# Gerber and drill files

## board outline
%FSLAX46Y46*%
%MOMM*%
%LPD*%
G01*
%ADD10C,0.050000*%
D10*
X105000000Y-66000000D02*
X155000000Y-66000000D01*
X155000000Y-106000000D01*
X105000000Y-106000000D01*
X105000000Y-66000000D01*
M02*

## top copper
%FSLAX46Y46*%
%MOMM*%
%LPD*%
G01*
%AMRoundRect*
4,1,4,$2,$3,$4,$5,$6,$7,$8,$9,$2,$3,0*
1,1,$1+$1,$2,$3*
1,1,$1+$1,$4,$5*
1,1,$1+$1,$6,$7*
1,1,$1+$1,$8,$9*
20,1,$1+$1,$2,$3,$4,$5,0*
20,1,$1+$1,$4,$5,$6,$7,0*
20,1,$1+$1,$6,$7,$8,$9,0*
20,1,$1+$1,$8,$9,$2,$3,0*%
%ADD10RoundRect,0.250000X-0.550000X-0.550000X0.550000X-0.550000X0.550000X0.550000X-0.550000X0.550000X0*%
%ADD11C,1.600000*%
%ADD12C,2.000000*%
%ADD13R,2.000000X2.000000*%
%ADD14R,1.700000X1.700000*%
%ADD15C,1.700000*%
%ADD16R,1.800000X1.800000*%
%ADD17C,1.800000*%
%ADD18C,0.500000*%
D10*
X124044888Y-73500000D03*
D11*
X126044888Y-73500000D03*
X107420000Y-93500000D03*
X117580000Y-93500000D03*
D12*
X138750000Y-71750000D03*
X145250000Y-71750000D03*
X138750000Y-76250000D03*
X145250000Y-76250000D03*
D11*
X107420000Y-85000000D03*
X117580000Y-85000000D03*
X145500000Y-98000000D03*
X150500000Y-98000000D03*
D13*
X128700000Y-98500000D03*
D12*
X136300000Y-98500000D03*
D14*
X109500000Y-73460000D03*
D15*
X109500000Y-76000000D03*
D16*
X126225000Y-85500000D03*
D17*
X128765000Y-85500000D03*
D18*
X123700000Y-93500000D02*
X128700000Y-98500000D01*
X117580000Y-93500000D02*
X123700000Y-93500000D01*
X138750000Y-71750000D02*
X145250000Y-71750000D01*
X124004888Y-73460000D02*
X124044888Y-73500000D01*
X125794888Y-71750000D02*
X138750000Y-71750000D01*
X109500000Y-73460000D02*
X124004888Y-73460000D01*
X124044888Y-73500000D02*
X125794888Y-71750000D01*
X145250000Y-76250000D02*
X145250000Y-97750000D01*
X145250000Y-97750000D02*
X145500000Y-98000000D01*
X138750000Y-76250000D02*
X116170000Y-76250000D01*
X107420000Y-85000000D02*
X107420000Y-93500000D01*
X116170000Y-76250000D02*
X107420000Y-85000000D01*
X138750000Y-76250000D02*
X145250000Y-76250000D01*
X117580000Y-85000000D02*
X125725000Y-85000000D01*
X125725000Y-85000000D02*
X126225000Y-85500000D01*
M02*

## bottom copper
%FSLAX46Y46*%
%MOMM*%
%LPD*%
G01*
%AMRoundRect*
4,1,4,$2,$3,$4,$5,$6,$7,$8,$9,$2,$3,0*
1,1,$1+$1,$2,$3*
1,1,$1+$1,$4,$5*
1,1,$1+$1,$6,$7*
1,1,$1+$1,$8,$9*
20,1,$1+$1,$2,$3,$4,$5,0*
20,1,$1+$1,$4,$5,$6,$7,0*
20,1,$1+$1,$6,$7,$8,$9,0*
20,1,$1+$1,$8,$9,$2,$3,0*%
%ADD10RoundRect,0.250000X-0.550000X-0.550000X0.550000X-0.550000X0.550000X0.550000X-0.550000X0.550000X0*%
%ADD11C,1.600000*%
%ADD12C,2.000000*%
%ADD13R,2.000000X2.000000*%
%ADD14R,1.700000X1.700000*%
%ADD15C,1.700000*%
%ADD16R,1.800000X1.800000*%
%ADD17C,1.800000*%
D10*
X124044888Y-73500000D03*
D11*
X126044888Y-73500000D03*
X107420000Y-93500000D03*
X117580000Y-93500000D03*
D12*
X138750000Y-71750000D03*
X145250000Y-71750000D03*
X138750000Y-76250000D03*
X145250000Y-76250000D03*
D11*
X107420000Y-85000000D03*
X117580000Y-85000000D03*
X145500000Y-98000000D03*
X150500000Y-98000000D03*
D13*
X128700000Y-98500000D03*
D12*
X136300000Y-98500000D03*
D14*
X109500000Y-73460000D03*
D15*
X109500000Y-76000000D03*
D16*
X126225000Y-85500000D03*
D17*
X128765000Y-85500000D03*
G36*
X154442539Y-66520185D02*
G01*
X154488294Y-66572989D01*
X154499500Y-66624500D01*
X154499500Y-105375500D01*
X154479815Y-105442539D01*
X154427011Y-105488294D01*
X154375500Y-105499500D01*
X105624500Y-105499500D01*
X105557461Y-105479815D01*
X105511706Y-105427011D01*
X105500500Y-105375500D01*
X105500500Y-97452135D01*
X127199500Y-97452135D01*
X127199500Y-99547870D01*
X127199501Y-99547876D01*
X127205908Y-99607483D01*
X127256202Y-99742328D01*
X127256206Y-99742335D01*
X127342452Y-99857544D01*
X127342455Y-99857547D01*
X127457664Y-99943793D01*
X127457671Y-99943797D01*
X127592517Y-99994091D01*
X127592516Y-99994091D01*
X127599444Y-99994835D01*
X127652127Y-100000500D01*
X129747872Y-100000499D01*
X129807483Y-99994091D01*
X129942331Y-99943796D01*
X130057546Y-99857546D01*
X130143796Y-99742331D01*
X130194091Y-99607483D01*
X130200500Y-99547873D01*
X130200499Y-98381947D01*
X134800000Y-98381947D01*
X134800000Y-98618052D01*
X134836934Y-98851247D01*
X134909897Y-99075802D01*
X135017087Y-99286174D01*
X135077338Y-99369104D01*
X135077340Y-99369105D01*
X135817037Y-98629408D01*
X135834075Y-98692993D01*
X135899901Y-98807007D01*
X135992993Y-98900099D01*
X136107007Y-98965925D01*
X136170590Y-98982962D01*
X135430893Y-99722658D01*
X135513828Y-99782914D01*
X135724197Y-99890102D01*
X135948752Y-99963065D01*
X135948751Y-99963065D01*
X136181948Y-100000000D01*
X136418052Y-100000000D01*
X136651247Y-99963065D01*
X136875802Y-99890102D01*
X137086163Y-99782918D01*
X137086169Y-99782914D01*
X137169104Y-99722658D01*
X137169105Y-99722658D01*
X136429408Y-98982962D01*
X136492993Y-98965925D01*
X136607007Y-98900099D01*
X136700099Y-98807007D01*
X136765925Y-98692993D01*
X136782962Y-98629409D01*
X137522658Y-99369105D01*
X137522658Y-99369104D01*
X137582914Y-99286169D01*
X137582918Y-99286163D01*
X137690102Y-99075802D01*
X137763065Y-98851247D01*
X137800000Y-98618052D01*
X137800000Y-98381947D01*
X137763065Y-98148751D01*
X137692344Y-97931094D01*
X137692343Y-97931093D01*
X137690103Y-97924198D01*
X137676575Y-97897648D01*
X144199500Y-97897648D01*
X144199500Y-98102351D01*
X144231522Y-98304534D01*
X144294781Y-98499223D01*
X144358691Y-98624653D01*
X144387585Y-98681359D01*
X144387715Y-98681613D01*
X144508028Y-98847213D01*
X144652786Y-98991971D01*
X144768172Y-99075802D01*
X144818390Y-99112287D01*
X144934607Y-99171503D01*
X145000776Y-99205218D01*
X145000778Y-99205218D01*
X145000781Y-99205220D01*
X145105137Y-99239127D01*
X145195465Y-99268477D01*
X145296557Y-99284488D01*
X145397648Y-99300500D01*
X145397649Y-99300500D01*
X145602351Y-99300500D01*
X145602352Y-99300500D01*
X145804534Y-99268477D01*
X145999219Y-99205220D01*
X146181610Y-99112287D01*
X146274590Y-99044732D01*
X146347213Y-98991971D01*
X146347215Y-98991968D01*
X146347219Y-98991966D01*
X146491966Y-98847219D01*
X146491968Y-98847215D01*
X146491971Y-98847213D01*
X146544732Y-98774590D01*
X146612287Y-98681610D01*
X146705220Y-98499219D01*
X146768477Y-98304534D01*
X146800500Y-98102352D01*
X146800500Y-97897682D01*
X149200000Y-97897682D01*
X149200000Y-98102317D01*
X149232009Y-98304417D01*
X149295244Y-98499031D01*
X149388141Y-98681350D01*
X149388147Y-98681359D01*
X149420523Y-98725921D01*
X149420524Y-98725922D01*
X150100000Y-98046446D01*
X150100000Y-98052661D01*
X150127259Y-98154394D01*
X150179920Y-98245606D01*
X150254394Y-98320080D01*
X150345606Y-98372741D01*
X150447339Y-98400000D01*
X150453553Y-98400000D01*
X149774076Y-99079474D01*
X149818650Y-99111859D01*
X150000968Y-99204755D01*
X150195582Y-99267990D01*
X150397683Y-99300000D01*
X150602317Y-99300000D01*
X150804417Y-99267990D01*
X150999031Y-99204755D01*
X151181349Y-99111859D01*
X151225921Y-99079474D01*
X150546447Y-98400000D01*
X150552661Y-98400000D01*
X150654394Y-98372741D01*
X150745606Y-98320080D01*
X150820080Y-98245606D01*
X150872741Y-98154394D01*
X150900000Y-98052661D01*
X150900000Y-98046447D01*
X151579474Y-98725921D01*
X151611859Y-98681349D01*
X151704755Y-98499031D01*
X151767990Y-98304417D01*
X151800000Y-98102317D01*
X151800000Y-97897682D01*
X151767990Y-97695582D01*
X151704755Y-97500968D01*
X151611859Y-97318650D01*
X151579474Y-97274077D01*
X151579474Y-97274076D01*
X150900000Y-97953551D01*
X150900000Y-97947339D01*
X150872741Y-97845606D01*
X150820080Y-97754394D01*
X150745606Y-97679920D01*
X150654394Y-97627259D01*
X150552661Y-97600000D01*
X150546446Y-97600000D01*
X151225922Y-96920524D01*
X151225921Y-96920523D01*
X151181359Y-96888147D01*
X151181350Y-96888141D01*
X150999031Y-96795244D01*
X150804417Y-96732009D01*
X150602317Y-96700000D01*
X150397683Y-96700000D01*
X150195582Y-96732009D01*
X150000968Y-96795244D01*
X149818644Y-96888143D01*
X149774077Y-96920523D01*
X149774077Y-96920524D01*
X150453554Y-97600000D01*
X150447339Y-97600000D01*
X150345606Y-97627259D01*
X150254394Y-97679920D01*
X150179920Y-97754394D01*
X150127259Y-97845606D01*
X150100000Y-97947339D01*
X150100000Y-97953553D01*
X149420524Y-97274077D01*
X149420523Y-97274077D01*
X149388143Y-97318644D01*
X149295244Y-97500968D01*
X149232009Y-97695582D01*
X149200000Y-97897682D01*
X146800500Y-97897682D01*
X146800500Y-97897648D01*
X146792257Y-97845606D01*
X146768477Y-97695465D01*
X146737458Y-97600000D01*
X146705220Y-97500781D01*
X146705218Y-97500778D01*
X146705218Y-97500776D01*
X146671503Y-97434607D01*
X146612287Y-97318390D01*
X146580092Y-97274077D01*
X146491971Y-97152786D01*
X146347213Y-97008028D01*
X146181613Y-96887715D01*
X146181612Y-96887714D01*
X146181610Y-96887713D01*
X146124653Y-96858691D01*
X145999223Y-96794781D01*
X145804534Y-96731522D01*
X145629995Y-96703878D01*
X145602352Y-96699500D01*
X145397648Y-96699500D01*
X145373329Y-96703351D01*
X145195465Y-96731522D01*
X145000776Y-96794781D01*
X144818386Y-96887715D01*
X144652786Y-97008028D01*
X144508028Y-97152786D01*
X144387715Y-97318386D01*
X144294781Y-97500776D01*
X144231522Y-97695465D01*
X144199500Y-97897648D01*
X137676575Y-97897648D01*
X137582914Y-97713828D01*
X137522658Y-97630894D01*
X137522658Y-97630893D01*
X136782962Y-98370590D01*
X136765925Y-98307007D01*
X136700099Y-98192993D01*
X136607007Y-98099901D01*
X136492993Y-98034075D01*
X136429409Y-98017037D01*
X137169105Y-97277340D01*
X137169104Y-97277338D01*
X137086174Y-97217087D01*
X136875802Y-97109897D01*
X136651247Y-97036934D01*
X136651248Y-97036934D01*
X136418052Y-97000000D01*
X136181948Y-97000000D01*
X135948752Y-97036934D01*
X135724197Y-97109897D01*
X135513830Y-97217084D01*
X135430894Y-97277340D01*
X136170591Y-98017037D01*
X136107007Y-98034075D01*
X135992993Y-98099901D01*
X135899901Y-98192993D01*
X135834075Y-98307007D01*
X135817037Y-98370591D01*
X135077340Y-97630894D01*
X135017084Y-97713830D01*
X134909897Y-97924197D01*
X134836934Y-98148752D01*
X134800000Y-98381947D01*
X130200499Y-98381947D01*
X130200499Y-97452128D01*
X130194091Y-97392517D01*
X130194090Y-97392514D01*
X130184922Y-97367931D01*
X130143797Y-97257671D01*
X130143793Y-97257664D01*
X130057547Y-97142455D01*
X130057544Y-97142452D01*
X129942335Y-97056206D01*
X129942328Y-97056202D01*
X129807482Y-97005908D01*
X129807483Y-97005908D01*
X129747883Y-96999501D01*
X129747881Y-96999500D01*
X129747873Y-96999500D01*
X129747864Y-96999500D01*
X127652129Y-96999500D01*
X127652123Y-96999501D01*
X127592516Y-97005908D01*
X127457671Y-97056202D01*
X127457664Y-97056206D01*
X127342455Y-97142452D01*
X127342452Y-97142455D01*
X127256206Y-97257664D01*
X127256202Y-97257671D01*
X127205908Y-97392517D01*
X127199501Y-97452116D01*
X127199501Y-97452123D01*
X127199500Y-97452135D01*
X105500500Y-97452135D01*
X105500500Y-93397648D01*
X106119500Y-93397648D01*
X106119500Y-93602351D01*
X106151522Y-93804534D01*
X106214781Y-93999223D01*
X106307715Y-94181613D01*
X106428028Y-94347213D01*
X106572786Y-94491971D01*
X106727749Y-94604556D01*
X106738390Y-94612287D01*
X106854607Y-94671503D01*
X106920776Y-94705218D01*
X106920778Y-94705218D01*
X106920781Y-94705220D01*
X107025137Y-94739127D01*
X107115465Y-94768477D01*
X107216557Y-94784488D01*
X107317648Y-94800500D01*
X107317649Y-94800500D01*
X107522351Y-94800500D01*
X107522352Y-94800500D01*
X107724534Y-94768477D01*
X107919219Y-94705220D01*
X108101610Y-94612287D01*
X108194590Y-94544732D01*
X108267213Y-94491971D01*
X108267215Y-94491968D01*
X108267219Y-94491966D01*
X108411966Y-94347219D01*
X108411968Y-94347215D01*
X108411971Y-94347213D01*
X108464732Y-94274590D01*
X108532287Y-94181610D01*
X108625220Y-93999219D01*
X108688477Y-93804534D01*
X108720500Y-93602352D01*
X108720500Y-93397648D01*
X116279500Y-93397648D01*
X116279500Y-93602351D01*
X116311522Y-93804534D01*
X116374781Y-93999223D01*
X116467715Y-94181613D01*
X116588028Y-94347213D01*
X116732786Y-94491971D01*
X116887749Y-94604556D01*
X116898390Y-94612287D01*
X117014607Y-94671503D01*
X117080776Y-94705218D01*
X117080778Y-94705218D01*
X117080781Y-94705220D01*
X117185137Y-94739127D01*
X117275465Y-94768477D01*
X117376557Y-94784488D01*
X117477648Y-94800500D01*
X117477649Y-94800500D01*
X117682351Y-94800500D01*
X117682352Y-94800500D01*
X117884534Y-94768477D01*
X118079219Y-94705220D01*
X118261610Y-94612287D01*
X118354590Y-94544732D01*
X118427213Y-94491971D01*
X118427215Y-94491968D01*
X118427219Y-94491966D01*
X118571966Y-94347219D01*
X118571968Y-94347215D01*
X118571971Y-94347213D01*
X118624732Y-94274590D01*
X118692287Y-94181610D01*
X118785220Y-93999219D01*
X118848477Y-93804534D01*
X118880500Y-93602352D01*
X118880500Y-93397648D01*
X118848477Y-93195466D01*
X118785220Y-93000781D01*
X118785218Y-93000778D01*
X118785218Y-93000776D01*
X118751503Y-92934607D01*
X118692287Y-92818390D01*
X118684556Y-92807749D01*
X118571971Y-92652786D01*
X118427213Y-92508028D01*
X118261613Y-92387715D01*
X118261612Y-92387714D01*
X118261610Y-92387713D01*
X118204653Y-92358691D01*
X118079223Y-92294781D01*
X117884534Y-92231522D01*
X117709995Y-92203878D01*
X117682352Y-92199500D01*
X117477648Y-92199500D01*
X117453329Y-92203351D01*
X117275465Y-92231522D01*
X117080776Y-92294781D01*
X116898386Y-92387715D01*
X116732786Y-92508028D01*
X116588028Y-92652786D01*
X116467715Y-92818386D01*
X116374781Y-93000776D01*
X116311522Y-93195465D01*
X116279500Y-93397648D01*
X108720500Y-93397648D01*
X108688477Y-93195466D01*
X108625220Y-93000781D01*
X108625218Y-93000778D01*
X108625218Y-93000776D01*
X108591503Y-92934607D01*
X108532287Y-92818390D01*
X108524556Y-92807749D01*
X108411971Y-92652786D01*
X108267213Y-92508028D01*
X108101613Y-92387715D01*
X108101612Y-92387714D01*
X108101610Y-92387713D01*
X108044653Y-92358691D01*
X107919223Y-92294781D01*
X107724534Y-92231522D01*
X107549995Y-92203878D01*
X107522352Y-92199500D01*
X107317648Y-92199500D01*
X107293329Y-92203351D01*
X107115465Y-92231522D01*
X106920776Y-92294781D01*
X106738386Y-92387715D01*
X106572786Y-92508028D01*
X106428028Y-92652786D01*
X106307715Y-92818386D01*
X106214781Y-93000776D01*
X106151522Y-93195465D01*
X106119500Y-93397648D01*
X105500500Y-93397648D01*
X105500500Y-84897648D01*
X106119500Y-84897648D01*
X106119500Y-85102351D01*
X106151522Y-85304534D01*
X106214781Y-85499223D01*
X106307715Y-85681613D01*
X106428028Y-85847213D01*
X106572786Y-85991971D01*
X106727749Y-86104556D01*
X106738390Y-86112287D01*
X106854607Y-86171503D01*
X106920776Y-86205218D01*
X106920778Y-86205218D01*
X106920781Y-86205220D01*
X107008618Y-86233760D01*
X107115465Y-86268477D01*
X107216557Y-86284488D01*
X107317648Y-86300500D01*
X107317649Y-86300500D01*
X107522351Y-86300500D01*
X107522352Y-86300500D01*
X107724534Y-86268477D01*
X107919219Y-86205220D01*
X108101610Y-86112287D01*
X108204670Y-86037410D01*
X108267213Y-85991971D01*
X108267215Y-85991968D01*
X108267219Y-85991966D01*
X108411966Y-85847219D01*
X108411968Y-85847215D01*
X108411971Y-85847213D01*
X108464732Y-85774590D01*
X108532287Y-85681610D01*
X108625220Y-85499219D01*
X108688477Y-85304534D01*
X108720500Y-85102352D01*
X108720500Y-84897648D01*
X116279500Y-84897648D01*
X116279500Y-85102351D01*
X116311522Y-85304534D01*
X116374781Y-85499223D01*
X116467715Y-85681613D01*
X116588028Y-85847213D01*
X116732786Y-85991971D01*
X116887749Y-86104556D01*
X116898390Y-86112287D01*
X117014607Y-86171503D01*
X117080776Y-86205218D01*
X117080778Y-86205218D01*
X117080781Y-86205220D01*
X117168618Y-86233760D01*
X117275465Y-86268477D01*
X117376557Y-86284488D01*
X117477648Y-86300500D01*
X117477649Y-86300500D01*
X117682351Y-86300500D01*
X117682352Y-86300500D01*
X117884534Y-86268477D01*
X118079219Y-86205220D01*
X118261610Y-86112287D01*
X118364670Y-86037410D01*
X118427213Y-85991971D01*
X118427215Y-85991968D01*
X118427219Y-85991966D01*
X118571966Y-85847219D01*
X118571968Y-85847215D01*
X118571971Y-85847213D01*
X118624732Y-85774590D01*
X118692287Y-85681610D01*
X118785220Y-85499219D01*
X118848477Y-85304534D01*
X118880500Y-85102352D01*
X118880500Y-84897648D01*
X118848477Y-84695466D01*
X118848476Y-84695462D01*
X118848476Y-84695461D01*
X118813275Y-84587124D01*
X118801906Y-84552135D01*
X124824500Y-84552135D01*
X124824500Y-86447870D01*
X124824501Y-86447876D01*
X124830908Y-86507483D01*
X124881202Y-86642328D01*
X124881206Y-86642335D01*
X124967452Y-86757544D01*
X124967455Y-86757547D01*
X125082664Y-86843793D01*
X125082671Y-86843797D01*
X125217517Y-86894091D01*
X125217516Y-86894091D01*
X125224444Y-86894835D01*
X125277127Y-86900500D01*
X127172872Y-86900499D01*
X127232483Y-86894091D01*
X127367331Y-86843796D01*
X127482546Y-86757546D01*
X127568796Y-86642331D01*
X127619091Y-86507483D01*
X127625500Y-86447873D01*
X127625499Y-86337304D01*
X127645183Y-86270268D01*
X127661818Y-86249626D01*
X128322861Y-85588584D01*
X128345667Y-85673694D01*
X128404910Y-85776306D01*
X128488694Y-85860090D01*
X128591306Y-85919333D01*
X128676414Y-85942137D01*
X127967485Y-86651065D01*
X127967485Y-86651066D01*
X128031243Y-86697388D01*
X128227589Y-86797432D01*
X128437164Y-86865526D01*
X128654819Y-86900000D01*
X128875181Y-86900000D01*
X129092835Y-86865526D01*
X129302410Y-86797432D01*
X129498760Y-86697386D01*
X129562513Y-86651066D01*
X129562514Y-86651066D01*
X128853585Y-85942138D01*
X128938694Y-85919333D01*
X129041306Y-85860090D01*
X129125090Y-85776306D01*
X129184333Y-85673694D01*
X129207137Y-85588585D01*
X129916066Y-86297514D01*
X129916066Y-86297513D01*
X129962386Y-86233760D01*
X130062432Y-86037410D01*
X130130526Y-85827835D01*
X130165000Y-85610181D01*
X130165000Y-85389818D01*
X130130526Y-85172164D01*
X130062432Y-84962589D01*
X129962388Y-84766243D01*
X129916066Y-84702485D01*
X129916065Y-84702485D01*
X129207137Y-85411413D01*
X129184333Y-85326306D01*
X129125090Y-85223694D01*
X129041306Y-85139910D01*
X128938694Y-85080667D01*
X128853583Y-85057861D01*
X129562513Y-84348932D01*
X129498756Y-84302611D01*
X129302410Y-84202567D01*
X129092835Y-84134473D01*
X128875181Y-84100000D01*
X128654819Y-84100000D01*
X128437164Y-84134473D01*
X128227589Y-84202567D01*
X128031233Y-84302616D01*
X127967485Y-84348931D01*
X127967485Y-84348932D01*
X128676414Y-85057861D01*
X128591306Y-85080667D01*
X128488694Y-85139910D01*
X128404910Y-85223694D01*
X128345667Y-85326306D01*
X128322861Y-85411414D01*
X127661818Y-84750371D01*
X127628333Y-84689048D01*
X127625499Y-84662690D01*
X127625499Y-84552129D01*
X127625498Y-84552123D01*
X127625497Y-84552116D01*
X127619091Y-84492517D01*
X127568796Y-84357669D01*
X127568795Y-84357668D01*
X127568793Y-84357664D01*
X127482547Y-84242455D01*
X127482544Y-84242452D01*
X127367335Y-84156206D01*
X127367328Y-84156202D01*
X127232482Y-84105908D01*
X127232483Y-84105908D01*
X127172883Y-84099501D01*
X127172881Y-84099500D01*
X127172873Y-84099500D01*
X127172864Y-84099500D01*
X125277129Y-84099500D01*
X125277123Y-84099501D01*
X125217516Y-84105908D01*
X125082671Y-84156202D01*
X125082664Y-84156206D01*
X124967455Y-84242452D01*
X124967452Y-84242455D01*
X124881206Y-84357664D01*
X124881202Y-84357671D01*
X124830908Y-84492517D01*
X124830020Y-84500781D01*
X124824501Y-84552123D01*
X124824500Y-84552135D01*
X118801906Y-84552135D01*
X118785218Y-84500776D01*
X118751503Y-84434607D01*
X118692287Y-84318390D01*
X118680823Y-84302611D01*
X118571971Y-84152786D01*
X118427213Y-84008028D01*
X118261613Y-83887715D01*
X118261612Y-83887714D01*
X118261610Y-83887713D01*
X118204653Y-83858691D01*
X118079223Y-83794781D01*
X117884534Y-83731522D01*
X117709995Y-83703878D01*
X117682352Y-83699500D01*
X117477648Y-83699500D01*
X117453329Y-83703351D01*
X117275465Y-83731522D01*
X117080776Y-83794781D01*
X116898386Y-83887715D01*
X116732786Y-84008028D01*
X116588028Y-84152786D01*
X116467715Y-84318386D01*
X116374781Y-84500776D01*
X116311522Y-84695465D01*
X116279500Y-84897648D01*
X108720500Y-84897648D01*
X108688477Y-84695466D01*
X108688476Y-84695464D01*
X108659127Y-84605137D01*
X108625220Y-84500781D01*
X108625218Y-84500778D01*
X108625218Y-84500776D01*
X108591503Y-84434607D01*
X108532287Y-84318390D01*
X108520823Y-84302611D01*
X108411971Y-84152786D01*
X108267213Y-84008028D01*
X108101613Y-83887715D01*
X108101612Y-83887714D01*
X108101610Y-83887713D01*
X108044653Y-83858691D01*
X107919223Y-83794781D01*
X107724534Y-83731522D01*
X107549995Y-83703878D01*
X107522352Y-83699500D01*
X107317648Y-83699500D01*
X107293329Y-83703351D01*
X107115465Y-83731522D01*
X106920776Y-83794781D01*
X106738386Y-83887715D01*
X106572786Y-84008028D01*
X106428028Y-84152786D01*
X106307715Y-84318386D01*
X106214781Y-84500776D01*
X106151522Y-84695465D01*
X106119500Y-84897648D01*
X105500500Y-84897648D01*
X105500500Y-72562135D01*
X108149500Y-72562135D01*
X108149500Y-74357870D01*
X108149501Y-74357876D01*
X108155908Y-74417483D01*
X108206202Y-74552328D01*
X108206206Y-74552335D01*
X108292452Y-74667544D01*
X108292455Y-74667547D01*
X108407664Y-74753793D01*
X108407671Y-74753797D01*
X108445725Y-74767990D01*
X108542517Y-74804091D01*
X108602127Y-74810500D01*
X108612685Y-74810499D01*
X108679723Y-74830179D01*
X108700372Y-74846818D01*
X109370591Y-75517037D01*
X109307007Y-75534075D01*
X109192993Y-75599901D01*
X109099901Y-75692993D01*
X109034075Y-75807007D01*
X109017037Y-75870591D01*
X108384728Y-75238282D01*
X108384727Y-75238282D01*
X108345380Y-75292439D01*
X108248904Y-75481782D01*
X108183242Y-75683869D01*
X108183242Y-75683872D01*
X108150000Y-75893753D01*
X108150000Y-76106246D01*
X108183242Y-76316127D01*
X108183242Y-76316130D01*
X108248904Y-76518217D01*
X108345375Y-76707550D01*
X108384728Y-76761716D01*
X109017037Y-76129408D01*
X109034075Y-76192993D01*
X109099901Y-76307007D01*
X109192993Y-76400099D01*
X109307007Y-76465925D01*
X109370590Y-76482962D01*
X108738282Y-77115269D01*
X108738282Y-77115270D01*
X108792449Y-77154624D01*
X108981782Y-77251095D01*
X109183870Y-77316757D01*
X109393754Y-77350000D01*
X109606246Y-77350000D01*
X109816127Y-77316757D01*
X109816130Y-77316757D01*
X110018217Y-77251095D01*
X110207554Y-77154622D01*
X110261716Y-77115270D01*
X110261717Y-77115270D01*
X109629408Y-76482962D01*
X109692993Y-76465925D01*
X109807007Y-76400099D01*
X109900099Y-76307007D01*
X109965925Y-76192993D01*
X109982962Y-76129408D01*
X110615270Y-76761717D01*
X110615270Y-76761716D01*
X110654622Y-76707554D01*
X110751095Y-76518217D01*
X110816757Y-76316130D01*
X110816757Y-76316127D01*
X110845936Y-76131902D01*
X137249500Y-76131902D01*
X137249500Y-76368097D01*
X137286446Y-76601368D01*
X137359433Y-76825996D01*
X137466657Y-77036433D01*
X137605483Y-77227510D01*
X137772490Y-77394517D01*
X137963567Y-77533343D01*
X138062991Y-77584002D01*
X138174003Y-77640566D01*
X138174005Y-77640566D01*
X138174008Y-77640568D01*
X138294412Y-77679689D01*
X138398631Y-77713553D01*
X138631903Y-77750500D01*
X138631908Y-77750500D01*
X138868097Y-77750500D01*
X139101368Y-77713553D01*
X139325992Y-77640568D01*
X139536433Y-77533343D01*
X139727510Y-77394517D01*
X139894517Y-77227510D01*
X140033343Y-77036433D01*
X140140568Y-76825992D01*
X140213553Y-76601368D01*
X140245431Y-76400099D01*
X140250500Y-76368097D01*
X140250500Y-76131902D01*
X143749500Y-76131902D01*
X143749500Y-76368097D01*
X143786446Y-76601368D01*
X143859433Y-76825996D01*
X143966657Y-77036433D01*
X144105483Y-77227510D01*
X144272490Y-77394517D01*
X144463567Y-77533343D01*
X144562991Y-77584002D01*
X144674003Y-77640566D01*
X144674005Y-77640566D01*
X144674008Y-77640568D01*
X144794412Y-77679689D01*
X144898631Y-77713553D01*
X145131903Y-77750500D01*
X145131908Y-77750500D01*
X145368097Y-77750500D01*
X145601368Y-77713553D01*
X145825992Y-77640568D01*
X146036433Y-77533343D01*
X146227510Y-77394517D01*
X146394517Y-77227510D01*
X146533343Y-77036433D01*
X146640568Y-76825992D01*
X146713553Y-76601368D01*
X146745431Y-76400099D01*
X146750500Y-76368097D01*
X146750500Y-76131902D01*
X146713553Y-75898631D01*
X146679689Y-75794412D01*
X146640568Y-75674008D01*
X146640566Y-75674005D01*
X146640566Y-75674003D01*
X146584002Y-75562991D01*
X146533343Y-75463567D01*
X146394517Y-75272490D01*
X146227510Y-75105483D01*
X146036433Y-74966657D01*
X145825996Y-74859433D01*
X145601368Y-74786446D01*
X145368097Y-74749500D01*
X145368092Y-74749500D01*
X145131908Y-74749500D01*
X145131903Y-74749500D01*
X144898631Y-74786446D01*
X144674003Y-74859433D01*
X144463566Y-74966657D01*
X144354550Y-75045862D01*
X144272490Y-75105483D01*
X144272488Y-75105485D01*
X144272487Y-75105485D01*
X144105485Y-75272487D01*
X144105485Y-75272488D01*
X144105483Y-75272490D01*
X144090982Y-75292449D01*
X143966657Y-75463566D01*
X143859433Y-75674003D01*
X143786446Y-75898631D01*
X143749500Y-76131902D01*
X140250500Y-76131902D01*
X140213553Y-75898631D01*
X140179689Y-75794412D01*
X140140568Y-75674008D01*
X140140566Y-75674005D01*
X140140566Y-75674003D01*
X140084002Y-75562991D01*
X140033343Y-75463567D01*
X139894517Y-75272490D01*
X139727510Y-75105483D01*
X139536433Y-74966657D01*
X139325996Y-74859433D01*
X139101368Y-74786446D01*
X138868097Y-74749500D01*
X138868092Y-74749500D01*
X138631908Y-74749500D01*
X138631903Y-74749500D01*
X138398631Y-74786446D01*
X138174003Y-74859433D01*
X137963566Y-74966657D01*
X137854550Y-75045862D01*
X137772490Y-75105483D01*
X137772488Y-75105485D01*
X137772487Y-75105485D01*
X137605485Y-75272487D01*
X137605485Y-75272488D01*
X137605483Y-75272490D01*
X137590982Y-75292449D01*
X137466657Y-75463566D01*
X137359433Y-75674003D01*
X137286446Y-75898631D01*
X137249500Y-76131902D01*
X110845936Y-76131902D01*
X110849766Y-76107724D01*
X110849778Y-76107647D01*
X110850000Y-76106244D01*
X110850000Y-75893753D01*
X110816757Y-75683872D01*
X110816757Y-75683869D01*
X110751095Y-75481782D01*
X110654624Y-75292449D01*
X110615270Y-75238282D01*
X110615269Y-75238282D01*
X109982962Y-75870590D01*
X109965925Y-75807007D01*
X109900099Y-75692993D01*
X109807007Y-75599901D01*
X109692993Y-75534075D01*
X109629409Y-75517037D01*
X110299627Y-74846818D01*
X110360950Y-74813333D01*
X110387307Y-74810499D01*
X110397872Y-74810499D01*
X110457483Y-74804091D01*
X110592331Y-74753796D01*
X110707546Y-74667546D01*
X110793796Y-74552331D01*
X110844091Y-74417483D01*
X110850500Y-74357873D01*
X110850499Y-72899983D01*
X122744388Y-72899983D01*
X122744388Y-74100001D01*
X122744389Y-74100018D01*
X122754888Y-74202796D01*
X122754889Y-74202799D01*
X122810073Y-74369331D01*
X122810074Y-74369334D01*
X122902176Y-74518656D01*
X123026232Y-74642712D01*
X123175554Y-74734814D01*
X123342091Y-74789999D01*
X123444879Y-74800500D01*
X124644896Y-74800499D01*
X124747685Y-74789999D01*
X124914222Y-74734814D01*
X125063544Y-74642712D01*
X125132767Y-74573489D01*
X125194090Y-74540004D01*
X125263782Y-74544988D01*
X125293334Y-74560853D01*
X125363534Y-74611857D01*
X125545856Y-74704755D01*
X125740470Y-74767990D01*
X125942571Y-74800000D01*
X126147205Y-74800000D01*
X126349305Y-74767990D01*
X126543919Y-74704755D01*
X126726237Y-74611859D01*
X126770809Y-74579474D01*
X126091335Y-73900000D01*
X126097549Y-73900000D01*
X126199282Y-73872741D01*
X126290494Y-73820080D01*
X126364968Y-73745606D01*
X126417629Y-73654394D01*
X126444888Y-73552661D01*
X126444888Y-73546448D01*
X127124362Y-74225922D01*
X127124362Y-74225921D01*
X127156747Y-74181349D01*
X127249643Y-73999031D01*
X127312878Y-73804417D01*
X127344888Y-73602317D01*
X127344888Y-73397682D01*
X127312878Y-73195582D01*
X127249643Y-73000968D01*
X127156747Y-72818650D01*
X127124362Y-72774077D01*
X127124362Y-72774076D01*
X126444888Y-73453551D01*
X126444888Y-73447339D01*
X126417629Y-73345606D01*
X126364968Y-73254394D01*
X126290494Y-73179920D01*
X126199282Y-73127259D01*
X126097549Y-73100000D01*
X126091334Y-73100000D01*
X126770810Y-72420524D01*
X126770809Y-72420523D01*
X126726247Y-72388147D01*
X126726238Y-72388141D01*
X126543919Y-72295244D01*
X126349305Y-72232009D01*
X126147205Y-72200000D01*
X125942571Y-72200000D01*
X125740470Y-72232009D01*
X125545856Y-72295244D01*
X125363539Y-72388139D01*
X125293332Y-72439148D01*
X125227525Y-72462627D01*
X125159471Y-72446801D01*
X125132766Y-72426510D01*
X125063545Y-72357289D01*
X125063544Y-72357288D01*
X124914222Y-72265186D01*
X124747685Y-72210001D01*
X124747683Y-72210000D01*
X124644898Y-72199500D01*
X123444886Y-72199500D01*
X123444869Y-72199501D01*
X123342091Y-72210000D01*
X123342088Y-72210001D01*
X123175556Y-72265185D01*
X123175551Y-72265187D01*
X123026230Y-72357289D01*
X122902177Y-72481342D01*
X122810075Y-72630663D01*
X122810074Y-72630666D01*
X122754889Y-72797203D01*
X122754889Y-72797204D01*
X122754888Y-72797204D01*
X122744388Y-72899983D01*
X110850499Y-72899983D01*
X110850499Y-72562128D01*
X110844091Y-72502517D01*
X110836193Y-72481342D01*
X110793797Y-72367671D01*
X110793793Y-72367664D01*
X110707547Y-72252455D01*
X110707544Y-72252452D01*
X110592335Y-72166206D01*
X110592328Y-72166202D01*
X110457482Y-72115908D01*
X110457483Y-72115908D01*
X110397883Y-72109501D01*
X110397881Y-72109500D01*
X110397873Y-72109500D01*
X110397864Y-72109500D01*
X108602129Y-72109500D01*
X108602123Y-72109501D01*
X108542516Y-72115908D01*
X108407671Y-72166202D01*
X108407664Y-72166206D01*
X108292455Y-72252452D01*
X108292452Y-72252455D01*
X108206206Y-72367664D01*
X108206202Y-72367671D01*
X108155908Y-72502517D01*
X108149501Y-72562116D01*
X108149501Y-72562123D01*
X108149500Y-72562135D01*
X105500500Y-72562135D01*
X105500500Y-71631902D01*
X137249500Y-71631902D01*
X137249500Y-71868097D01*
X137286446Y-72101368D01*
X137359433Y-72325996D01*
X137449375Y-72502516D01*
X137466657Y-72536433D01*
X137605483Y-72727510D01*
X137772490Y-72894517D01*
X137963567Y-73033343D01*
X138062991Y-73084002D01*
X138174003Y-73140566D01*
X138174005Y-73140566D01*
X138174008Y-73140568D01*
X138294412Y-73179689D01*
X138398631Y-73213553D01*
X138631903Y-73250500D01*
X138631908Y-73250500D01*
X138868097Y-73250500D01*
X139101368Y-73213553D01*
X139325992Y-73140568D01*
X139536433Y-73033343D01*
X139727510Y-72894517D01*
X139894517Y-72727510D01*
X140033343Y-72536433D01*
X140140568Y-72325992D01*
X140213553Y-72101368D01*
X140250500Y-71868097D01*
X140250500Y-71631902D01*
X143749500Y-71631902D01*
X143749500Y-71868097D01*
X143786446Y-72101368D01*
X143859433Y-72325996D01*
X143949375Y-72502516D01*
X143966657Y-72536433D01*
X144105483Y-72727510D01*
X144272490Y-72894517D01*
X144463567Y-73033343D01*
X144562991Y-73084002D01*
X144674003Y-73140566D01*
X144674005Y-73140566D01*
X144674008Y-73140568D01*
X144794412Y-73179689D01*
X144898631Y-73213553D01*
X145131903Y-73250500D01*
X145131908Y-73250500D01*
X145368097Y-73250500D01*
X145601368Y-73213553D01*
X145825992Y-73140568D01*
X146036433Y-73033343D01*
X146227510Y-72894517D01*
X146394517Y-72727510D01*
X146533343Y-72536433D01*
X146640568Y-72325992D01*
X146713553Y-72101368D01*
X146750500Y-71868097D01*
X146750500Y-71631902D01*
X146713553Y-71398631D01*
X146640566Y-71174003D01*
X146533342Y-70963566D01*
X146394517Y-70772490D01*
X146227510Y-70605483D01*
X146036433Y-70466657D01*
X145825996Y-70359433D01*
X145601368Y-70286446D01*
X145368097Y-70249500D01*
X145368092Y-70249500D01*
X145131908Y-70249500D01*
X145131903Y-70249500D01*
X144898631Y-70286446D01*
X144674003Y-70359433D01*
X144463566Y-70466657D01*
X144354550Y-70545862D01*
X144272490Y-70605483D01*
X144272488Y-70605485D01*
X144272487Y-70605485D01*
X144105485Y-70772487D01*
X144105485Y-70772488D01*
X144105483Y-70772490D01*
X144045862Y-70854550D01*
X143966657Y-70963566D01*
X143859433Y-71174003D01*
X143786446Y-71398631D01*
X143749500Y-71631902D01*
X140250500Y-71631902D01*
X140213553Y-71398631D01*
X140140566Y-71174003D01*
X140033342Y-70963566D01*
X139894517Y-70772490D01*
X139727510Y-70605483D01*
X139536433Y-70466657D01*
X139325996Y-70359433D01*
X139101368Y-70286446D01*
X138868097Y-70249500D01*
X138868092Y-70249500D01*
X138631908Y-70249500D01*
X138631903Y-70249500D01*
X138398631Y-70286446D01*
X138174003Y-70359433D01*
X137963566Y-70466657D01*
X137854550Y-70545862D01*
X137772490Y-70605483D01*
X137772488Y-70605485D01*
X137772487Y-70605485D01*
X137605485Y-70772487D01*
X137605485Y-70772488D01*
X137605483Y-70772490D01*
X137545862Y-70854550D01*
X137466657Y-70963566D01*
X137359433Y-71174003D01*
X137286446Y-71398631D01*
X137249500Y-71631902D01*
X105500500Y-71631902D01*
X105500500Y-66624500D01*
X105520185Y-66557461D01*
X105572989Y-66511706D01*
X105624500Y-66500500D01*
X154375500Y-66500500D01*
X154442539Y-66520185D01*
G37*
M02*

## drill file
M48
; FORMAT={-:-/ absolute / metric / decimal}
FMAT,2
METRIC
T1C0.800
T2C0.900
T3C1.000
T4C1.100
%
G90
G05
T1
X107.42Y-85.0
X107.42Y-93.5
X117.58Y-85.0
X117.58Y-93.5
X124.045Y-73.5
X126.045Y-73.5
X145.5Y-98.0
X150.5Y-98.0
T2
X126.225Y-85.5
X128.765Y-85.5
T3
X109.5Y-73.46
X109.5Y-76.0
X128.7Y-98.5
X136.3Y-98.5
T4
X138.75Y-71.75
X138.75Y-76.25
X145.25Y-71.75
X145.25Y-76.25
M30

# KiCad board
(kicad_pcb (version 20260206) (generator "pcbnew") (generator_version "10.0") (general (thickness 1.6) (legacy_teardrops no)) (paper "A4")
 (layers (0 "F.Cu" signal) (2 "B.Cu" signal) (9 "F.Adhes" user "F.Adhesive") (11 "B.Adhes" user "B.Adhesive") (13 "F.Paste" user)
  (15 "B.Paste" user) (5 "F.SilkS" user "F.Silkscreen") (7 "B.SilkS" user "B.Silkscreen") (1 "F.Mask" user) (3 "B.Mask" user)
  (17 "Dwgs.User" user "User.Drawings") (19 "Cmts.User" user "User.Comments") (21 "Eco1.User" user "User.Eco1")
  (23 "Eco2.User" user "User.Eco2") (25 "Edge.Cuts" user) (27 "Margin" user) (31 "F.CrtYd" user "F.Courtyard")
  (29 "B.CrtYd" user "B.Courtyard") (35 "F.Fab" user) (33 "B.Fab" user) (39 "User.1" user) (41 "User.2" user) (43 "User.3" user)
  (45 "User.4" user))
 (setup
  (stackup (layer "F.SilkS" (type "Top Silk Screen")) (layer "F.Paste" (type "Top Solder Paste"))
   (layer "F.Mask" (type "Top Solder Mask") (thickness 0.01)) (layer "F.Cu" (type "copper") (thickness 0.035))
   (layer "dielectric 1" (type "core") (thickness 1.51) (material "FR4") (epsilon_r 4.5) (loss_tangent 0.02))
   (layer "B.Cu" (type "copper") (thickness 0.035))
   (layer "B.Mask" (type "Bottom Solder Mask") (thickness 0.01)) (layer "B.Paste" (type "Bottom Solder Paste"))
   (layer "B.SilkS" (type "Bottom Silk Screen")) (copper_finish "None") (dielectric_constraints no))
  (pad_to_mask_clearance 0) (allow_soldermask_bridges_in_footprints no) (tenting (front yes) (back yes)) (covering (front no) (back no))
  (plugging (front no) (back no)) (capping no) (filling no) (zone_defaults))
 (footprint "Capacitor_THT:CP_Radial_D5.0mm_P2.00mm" (layer "F.Cu") (at 124.044888 73.5)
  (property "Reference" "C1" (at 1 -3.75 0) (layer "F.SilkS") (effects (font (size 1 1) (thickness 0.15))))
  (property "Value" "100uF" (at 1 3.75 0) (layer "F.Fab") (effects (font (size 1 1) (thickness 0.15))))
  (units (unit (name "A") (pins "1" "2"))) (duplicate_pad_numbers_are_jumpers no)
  (pad "1" thru_hole roundrect (at 0 0) (size 1.6 1.6) (drill 0.8) (layers "*.Cu" "*.Mask") (remove_unused_layers no)
   (roundrect_rratio 0.15625) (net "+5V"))
  (pad "2" thru_hole circle (at 2 0) (size 1.6 1.6) (drill 0.8) (layers "*.Cu" "*.Mask") (remove_unused_layers no) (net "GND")))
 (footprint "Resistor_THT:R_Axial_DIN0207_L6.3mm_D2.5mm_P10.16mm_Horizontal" (layer "F.Cu") (at 107.42 93.5)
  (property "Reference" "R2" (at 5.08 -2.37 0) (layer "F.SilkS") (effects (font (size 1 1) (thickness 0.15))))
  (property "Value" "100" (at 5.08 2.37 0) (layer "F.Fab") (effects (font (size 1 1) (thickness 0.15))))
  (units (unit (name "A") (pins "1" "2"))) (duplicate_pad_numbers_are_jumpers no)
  (pad "1" thru_hole circle (at 0 0) (size 1.6 1.6) (drill 0.8) (layers "*.Cu" "*.Mask") (remove_unused_layers no) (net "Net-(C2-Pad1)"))
  (pad "2" thru_hole circle (at 10.16 0) (size 1.6 1.6) (drill 0.8) (layers "*.Cu" "*.Mask") (remove_unused_layers no) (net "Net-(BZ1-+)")))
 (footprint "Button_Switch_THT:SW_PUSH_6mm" (layer "F.Cu") (at 138.75 71.75)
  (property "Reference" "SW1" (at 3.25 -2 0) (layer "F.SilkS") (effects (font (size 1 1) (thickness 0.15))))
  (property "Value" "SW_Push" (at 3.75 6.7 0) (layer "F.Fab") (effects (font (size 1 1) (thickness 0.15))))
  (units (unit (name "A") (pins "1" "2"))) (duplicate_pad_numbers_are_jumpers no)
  (pad "1" thru_hole circle (at 0 0 90) (size 2 2) (drill 1.1) (layers "*.Cu" "*.Mask") (remove_unused_layers no) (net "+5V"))
  (pad "1" thru_hole circle (at 6.5 0 90) (size 2 2) (drill 1.1) (layers "*.Cu" "*.Mask") (remove_unused_layers no) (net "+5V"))
  (pad "2" thru_hole circle (at 0 4.5 90) (size 2 2) (drill 1.1) (layers "*.Cu" "*.Mask") (remove_unused_layers no) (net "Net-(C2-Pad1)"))
  (pad "2" thru_hole circle (at 6.5 4.5 90) (size 2 2) (drill 1.1) (layers "*.Cu" "*.Mask") (remove_unused_layers no) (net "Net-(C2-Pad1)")))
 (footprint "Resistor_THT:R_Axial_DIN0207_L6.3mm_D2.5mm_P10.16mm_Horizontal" (layer "F.Cu") (at 107.42 85)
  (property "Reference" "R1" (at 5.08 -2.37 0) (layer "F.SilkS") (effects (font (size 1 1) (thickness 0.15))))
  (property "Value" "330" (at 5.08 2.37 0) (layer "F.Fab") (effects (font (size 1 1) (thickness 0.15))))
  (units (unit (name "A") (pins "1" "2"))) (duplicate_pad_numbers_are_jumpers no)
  (pad "1" thru_hole circle (at 0 0) (size 1.6 1.6) (drill 0.8) (layers "*.Cu" "*.Mask") (remove_unused_layers no) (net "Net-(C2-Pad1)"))
  (pad "2" thru_hole circle (at 10.16 0) (size 1.6 1.6) (drill 0.8) (layers "*.Cu" "*.Mask") (remove_unused_layers no) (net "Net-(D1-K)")))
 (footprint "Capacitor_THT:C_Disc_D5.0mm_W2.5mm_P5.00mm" (layer "F.Cu") (at 145.5 98)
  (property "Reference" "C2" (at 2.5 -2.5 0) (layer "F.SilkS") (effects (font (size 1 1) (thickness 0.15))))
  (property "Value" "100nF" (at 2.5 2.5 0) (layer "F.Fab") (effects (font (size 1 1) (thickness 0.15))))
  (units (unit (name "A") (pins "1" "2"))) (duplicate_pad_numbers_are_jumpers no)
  (pad "1" thru_hole circle (at 0 0) (size 1.6 1.6) (drill 0.8) (layers "*.Cu" "*.Mask") (remove_unused_layers no) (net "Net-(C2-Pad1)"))
  (pad "2" thru_hole circle (at 5 0) (size 1.6 1.6) (drill 0.8) (layers "*.Cu" "*.Mask") (remove_unused_layers no) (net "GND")))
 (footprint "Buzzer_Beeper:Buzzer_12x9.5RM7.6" (layer "F.Cu") (at 128.7 98.5)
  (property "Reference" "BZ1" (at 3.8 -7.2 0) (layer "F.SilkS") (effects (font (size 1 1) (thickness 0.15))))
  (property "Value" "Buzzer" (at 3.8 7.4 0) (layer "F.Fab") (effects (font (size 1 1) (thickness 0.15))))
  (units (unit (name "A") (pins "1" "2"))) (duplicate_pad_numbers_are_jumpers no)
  (pad "1" thru_hole rect (at 0 0) (size 2 2) (drill 1) (layers "*.Cu" "*.Mask") (remove_unused_layers no) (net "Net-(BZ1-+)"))
  (pad "2" thru_hole circle (at 7.6 0) (size 2 2) (drill 1) (layers "*.Cu" "*.Mask") (remove_unused_layers no) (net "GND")))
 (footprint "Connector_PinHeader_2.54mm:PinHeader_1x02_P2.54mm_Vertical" (layer "F.Cu") (at 109.5 73.46)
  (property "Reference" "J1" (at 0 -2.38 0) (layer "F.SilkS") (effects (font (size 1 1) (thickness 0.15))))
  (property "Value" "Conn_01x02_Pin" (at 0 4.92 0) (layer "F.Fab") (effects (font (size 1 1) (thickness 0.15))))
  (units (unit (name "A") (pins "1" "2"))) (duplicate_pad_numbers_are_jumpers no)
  (pad "1" thru_hole rect (at 0 0) (size 1.7 1.7) (drill 1) (layers "*.Cu" "*.Mask") (remove_unused_layers no) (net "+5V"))
  (pad "2" thru_hole circle (at 0 2.54) (size 1.7 1.7) (drill 1) (layers "*.Cu" "*.Mask") (remove_unused_layers no) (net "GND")))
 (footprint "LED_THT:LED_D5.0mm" (layer "F.Cu") (at 126.225 85.5)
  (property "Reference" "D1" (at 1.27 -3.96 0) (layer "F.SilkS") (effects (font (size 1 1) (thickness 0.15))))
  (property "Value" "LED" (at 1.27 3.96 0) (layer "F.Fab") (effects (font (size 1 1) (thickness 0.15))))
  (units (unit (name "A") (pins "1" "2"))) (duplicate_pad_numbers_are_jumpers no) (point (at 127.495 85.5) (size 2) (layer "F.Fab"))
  (pad "1" thru_hole rect (at 0 0) (size 1.8 1.8) (drill 0.9) (layers "*.Cu" "*.Mask") (remove_unused_layers no) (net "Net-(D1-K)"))
  (pad "2" thru_hole circle (at 2.54 0) (size 1.8 1.8) (drill 0.9) (layers "*.Cu" "*.Mask") (remove_unused_layers no) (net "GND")))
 (gr_rect (start 105 66) (end 155 106) (stroke (width 0.05) (type default)) (fill no) (layer "Edge.Cuts"))
 (segment (start 123.7 93.5) (end 128.7 98.5) (width 0.5) (layer "F.Cu") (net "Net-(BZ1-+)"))
 (segment (start 117.58 93.5) (end 123.7 93.5) (width 0.5) (layer "F.Cu") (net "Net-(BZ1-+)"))
 (segment (start 138.75 71.75) (end 145.25 71.75) (width 0.5) (layer "F.Cu") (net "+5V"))
 (segment (start 124.004888 73.46) (end 124.044888 73.5) (width 0.5) (layer "F.Cu") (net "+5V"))
 (segment (start 125.794888 71.75) (end 138.75 71.75) (width 0.5) (layer "F.Cu") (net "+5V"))
 (segment (start 109.5 73.46) (end 124.004888 73.46) (width 0.5) (layer "F.Cu") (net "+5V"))
 (segment (start 124.044888 73.5) (end 125.794888 71.75) (width 0.5) (layer "F.Cu") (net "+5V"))
 (segment (start 145.25 76.25) (end 145.25 97.75) (width 0.5) (layer "F.Cu") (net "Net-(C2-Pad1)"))
 (segment (start 145.25 97.75) (end 145.5 98) (width 0.5) (layer "F.Cu") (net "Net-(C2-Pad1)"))
 (segment (start 138.75 76.25) (end 116.17 76.25) (width 0.5) (layer "F.Cu") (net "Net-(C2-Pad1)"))
 (segment (start 107.42 85) (end 107.42 93.5) (width 0.5) (layer "F.Cu") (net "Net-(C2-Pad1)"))
 (segment (start 116.17 76.25) (end 107.42 85) (width 0.5) (layer "F.Cu") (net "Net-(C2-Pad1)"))
 (segment (start 138.75 76.25) (end 145.25 76.25) (width 0.5) (layer "F.Cu") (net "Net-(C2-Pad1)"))
 (segment (start 117.58 85) (end 125.725 85) (width 0.5) (layer "F.Cu") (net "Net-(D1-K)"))
 (segment (start 125.725 85) (end 126.225 85.5) (width 0.5) (layer "F.Cu") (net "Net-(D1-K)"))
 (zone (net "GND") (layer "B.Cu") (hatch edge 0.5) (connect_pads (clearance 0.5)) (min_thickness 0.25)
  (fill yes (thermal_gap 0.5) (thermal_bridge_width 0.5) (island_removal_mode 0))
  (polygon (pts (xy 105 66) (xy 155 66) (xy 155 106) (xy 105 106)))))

